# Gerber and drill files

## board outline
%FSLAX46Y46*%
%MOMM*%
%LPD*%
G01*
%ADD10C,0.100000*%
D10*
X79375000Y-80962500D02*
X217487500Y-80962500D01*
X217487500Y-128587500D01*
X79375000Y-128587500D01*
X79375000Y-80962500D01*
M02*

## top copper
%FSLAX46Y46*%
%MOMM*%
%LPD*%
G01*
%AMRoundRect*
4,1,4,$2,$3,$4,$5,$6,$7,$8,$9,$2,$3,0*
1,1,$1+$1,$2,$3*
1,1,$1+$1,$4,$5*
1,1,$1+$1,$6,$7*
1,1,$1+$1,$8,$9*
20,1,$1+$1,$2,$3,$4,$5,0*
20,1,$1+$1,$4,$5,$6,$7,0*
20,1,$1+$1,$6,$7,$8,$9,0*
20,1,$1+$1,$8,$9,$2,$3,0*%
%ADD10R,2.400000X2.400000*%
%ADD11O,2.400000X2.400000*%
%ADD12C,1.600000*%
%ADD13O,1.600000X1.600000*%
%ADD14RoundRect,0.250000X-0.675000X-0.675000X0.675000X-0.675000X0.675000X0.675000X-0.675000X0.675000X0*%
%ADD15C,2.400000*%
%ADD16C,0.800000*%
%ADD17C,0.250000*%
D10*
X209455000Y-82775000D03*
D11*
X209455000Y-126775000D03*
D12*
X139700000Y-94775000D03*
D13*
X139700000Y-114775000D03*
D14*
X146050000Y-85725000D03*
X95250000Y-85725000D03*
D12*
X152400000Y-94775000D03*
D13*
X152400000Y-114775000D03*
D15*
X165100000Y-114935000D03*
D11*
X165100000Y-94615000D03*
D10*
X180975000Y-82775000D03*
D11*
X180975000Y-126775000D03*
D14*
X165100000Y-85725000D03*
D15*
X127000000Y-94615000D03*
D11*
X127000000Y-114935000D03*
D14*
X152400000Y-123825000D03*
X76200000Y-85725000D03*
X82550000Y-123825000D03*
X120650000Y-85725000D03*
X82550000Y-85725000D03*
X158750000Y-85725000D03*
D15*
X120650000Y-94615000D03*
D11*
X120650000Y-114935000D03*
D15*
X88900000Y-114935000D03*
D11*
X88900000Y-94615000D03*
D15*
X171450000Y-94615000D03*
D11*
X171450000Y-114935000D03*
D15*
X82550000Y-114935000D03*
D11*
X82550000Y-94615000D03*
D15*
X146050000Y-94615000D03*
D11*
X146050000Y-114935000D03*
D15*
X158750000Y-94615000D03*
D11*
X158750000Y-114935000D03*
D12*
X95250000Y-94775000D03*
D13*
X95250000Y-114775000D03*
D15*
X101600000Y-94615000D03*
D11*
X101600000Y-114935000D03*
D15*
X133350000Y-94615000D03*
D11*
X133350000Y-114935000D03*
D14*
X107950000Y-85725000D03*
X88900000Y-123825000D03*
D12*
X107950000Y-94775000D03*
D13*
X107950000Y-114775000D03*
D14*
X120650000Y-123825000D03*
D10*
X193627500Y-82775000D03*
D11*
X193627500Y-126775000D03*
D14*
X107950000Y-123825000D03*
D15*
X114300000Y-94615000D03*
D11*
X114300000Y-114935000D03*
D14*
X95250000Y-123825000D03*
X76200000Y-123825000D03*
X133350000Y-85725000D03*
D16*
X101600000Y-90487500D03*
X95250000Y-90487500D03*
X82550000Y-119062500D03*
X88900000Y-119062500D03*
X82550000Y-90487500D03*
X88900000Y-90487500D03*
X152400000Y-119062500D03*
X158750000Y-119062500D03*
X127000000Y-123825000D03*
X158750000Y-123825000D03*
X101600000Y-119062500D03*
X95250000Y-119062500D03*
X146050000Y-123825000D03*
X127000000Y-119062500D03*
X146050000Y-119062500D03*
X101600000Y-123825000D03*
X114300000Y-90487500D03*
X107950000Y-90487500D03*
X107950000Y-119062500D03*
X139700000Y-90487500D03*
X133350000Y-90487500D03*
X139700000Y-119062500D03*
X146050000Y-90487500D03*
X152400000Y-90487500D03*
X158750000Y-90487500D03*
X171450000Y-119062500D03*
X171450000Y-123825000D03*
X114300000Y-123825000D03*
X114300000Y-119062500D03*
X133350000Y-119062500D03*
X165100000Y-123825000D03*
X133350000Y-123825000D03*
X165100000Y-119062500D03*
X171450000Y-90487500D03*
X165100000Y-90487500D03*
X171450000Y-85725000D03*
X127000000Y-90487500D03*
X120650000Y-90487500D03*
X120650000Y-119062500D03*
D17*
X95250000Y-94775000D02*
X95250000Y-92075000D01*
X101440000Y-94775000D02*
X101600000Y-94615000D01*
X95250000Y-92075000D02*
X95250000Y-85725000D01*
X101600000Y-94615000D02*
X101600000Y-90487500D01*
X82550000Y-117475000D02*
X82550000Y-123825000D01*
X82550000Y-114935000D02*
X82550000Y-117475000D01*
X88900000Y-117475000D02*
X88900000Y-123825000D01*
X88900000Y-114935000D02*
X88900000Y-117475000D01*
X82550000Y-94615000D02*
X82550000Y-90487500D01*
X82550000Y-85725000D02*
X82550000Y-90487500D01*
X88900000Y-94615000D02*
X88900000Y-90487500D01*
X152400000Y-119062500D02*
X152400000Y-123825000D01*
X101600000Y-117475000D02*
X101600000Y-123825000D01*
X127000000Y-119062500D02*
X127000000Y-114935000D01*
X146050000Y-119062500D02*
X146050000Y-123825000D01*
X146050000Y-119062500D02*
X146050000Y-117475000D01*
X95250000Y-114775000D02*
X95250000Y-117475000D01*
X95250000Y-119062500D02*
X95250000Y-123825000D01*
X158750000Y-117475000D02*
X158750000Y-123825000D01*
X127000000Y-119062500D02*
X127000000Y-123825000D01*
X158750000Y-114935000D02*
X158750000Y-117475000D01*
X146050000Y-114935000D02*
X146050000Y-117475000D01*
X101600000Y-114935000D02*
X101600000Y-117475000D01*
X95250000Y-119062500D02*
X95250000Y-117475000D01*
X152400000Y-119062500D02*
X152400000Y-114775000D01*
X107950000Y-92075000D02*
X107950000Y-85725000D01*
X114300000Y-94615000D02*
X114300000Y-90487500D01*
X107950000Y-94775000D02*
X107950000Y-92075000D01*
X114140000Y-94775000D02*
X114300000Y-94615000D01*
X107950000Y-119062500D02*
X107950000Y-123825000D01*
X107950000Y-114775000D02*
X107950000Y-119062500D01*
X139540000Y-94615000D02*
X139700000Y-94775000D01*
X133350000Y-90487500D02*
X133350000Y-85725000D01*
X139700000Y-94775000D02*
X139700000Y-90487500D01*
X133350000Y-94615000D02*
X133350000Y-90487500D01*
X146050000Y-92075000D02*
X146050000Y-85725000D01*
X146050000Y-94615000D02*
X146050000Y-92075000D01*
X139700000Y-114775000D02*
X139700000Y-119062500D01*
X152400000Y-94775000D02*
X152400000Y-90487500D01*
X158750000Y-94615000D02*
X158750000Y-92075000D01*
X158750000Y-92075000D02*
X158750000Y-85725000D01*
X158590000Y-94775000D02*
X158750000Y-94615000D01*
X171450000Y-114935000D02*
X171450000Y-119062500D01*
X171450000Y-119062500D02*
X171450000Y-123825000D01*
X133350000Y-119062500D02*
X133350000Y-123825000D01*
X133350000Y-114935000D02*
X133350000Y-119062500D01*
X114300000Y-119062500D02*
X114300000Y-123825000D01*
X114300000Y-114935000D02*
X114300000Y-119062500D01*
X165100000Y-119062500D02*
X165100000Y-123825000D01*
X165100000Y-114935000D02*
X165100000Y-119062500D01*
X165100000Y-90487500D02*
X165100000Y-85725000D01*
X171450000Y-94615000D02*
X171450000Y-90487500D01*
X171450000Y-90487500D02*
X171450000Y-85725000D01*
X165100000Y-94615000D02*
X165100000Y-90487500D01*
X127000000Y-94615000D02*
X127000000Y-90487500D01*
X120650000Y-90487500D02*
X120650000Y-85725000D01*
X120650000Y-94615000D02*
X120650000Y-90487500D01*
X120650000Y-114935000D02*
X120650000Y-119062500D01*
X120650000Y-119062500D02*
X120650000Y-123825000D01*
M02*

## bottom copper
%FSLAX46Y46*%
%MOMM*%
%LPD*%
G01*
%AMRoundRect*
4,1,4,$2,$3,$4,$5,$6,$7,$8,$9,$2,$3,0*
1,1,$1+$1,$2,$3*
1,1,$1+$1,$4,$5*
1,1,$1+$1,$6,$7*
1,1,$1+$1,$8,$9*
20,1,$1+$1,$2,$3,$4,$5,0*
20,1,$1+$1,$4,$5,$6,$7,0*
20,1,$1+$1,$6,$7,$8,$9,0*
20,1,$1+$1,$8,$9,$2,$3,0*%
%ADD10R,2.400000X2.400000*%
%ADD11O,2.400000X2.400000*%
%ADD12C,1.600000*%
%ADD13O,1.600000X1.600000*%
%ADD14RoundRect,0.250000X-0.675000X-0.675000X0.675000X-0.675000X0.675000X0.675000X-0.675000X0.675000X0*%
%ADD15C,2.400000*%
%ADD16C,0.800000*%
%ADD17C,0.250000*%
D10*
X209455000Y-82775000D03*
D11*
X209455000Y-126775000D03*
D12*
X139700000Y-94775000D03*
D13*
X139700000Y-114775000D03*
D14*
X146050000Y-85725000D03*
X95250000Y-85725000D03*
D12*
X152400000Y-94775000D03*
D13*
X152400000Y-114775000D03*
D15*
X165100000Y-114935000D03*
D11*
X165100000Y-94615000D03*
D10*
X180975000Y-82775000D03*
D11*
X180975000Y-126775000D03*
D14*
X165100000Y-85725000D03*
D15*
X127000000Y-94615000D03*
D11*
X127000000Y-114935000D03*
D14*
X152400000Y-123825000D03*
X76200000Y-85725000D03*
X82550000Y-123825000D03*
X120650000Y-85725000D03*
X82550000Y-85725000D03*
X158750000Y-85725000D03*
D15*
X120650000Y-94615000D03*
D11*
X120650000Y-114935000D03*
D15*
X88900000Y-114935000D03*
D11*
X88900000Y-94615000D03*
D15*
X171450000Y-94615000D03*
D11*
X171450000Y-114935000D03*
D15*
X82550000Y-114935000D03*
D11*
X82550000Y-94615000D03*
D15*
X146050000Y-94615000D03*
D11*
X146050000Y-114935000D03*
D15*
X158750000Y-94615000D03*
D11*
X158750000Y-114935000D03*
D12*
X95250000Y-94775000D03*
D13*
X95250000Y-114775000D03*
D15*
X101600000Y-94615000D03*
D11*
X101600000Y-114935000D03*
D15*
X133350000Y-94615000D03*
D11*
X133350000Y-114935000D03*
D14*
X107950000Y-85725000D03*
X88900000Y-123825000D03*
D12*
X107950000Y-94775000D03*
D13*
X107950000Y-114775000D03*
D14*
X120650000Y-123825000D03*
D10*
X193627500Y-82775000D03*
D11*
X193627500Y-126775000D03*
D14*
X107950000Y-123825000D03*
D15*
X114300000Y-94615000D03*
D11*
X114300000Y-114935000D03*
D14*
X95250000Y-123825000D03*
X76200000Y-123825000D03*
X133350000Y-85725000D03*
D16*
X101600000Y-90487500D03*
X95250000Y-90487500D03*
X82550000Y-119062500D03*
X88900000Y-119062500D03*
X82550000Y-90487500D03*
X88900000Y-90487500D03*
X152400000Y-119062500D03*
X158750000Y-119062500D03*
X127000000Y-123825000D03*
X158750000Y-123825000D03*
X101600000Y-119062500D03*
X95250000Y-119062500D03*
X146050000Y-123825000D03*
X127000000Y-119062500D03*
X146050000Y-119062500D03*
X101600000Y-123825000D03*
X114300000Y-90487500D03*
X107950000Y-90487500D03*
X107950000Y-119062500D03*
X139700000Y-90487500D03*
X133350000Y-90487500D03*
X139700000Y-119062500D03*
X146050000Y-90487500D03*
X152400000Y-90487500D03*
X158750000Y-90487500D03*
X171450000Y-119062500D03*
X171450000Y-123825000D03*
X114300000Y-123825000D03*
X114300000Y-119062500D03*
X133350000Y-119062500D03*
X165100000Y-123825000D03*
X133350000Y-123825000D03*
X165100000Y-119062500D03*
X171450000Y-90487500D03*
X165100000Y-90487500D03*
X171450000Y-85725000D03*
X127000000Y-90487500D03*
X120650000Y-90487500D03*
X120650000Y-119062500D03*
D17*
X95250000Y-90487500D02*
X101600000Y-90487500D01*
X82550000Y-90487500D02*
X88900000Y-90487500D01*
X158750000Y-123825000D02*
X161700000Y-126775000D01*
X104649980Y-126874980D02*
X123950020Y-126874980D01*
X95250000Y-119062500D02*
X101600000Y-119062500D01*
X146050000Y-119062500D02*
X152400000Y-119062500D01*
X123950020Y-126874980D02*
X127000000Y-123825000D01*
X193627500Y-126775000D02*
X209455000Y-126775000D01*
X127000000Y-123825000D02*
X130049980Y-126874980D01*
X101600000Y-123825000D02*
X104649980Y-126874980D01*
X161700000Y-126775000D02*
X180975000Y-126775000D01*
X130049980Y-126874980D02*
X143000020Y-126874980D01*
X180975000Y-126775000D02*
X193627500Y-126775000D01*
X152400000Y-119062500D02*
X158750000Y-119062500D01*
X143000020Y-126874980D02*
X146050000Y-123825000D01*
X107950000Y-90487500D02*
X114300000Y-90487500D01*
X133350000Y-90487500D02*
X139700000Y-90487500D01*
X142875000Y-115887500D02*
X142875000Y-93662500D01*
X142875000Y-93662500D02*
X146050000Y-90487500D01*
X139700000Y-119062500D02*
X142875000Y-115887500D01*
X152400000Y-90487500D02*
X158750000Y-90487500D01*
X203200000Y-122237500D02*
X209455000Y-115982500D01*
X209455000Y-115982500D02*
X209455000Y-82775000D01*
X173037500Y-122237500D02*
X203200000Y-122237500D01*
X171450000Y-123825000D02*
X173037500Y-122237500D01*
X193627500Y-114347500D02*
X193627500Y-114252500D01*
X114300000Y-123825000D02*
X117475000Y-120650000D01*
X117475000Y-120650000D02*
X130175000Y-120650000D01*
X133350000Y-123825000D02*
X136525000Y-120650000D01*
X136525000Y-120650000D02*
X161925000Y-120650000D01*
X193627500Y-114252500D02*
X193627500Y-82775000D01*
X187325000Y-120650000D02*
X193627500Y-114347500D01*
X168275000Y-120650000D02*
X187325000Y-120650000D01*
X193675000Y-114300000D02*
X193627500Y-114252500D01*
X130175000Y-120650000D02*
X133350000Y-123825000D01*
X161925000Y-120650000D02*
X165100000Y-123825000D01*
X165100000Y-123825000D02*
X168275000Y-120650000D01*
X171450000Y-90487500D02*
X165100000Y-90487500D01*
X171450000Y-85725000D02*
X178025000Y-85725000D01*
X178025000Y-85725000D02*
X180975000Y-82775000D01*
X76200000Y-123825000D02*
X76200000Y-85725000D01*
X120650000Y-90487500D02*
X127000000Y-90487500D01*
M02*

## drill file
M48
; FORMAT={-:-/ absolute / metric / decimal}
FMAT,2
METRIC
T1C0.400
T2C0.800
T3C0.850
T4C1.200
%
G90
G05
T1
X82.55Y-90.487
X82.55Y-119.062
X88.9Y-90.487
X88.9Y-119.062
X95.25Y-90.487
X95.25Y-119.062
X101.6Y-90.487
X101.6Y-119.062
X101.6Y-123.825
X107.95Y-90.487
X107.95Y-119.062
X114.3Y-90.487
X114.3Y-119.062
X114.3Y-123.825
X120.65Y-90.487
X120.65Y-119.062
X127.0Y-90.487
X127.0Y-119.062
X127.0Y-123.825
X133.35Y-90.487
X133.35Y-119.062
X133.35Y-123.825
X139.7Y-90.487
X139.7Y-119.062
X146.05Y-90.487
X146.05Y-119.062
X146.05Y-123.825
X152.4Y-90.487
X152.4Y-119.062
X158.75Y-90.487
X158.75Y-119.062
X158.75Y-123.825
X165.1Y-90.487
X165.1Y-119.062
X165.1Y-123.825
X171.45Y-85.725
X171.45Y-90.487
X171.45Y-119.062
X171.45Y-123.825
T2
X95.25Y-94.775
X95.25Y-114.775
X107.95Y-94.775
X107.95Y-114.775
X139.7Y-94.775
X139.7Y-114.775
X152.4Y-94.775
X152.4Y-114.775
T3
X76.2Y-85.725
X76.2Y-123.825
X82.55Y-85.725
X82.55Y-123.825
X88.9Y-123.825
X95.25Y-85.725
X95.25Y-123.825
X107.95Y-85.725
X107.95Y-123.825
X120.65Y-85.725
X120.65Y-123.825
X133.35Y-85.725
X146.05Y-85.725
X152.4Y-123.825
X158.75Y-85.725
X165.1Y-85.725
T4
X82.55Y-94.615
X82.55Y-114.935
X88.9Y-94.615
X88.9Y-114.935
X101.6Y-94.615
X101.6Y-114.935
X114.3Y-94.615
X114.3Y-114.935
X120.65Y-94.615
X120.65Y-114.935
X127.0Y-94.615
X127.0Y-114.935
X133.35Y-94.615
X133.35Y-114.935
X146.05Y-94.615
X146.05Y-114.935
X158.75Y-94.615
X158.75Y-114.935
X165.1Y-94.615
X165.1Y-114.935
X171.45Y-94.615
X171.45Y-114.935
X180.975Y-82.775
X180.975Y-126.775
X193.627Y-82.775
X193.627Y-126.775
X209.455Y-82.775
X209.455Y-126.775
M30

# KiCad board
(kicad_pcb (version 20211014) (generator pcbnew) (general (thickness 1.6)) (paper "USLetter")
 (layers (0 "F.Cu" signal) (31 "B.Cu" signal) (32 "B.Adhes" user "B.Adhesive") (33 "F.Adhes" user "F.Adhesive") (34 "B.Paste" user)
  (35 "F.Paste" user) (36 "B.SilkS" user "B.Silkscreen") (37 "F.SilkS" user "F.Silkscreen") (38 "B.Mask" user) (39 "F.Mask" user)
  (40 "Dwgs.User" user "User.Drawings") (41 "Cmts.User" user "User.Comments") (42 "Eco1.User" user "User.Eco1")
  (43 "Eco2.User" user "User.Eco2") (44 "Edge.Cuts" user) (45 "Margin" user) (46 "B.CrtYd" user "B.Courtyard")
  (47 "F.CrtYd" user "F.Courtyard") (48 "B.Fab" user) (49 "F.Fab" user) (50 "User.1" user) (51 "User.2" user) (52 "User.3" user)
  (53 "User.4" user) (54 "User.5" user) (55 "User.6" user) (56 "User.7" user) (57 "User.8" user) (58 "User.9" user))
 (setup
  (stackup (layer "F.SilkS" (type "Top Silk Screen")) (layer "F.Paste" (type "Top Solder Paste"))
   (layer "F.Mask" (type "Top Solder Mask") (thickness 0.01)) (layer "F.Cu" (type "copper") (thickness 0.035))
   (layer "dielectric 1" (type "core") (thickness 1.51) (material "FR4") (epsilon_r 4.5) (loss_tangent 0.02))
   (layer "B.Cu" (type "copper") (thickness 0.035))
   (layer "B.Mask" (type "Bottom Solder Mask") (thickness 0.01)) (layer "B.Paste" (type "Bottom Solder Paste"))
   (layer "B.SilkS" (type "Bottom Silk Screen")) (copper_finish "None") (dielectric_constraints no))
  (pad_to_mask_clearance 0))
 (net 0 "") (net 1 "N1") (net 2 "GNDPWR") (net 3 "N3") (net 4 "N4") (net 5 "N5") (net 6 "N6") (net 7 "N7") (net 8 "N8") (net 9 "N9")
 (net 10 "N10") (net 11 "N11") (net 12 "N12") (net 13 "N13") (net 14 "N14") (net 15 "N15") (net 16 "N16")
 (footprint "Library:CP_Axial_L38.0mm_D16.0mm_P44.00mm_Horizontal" (layer "F.Cu") (at 209.455 82.775 -90)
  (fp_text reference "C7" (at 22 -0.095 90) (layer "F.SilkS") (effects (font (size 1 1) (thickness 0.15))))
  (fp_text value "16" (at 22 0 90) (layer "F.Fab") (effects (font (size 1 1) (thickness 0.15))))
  (pad "1" thru_hole rect (at 0 0 270) (size 2.4 2.4) (drill 1.2) (layers *.Cu *.Mask) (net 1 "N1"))
  (pad "2" thru_hole oval (at 44 0 270) (size 2.4 2.4) (drill 1.2) (layers *.Cu *.Mask) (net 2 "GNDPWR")))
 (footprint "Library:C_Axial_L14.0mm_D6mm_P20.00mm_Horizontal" (layer "F.Cu") (at 139.7 94.775 -90)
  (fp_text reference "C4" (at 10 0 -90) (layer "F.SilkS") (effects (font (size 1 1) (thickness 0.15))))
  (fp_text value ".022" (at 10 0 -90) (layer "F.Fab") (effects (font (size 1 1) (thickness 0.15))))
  (pad "1" thru_hole circle (at 0 0 270) (size 1.6 1.6) (drill 0.8) (layers *.Cu *.Mask) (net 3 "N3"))
  (pad "2" thru_hole oval (at 20 0 270) (size 1.6 1.6) (drill 0.8) (layers *.Cu *.Mask) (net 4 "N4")))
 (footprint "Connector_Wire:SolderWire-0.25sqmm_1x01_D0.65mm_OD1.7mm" (layer "F.Cu") (at 146.05 85.725)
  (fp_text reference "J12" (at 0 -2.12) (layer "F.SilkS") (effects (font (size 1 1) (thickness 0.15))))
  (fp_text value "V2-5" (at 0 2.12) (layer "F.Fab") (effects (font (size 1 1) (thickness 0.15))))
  (pad "1" thru_hole roundrect (at 0 0) (size 1.85 1.85) (drill 0.85) (layers *.Cu *.Mask) (roundrect_rratio 0.135135) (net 4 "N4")))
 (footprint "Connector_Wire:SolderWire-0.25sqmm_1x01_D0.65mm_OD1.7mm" (layer "F.Cu") (at 95.25 85.725)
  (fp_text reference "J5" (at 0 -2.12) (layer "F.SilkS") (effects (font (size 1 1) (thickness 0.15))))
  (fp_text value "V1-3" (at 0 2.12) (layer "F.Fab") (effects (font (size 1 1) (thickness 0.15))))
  (pad "1" thru_hole roundrect (at 0 0) (size 1.85 1.85) (drill 0.85) (layers *.Cu *.Mask) (roundrect_rratio 0.135135) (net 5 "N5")))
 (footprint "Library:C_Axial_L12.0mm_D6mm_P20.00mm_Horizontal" (layer "F.Cu") (at 152.4 94.775 -90)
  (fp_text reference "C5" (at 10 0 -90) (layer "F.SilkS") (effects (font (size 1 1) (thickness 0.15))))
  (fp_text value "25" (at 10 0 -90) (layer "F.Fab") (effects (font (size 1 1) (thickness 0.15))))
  (pad "1" thru_hole circle (at 0 0 270) (size 1.6 1.6) (drill 0.8) (layers *.Cu *.Mask) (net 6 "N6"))
  (pad "2" thru_hole oval (at 20 0 270) (size 1.6 1.6) (drill 0.8) (layers *.Cu *.Mask) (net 2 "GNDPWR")))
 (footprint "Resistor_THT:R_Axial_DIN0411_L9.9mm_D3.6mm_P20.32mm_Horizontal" (layer "F.Cu") (at 165.1 114.935 90)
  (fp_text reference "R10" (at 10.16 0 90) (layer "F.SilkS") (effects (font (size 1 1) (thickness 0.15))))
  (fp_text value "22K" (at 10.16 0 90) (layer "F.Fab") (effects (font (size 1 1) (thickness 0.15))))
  (pad "1" thru_hole circle (at 0 0 90) (size 2.4 2.4) (drill 1.2) (layers *.Cu *.Mask) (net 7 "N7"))
  (pad "2" thru_hole oval (at 20.32 0 90) (size 2.4 2.4) (drill 1.2) (layers *.Cu *.Mask) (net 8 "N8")))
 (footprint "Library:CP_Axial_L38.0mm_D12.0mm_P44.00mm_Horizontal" (layer "F.Cu") (at 180.975 82.775 -90)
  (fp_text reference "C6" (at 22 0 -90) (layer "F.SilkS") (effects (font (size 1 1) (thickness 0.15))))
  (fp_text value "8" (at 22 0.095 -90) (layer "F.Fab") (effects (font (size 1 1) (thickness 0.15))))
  (pad "1" thru_hole rect (at 0 0 270) (size 2.4 2.4) (drill 1.2) (layers *.Cu *.Mask) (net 8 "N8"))
  (pad "2" thru_hole oval (at 44 0 270) (size 2.4 2.4) (drill 1.2) (layers *.Cu *.Mask) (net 2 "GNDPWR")))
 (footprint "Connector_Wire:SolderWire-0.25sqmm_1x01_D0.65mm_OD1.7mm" (layer "F.Cu") (at 165.1 85.725)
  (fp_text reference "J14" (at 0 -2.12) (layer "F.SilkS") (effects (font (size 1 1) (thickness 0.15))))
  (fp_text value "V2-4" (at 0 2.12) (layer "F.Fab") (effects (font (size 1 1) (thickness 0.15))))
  (pad "1" thru_hole roundrect (at 0 0) (size 1.85 1.85) (drill 0.85) (layers *.Cu *.Mask) (roundrect_rratio 0.135135) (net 8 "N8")))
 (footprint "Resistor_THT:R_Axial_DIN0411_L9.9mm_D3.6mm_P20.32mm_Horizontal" (layer "F.Cu") (at 127 94.615 -90)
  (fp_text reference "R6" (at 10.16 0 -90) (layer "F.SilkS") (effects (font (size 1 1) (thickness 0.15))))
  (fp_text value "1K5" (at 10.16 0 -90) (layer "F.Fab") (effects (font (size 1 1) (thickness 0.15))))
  (pad "1" thru_hole circle (at 0 0 270) (size 2.4 2.4) (drill 1.2) (layers *.Cu *.Mask) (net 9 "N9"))
  (pad "2" thru_hole oval (at 20.32 0 270) (size 2.4 2.4) (drill 1.2) (layers *.Cu *.Mask) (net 2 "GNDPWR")))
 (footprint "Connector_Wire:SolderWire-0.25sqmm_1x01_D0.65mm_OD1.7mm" (layer "F.Cu") (at 152.4 123.825)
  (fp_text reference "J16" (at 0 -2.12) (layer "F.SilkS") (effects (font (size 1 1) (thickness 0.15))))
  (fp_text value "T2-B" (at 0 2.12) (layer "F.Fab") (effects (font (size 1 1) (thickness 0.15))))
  (pad "1" thru_hole roundrect (at 0 0) (size 1.85 1.85) (drill 0.85) (layers *.Cu *.Mask) (roundrect_rratio 0.135135) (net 2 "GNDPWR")))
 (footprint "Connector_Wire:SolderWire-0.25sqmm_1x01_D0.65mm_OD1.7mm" (layer "F.Cu") (at 76.2 85.725)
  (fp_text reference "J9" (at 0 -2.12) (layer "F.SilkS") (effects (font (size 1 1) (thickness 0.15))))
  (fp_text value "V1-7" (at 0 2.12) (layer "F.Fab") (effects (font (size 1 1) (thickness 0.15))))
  (pad "1" thru_hole roundrect (at 0 0) (size 1.85 1.85) (drill 0.85) (layers *.Cu *.Mask) (roundrect_rratio 0.135135) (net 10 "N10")))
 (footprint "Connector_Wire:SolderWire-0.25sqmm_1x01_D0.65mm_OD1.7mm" (layer "F.Cu") (at 82.55 123.825)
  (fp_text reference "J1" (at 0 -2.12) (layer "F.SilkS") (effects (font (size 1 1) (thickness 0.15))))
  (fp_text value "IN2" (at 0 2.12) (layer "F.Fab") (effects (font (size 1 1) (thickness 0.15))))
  (pad "1" thru_hole roundrect (at 0 0) (size 1.85 1.85) (drill 0.85) (layers *.Cu *.Mask) (roundrect_rratio 0.135135) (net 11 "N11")))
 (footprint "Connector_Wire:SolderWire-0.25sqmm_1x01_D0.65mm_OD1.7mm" (layer "F.Cu") (at 120.65 85.725)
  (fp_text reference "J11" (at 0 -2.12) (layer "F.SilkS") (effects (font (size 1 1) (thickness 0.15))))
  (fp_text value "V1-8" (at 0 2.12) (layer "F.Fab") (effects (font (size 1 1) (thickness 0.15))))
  (pad "1" thru_hole roundrect (at 0 0) (size 1.85 1.85) (drill 0.85) (layers *.Cu *.Mask) (roundrect_rratio 0.135135) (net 9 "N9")))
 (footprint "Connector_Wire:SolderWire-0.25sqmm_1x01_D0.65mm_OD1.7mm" (layer "F.Cu") (at 82.55 85.725)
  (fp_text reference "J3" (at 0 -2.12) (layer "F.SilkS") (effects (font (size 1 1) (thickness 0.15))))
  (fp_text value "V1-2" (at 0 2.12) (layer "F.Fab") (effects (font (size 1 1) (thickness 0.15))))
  (pad "1" thru_hole roundrect (at 0 0) (size 1.85 1.85) (drill 0.85) (layers *.Cu *.Mask) (roundrect_rratio 0.135135) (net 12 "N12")))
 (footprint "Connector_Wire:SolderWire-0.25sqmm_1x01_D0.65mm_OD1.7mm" (layer "F.Cu") (at 158.75 85.725)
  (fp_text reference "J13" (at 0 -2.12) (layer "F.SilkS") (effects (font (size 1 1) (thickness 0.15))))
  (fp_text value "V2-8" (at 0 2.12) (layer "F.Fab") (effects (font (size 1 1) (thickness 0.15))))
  (pad "1" thru_hole roundrect (at 0 0) (size 1.85 1.85) (drill 0.85) (layers *.Cu *.Mask) (roundrect_rratio 0.135135) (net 6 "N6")))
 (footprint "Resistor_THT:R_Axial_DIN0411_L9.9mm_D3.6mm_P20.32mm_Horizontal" (layer "F.Cu") (at 120.65 94.615 -90)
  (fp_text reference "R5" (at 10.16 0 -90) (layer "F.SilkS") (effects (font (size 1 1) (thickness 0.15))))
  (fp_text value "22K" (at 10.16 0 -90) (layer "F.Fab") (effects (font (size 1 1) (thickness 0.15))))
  (pad "1" thru_hole circle (at 0 0 270) (size 2.4 2.4) (drill 1.2) (layers *.Cu *.Mask) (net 9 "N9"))
  (pad "2" thru_hole oval (at 20.32 0 270) (size 2.4 2.4) (drill 1.2) (layers *.Cu *.Mask) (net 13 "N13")))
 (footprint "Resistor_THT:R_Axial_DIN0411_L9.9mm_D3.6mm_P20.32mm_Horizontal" (layer "F.Cu") (at 88.9 114.935 90)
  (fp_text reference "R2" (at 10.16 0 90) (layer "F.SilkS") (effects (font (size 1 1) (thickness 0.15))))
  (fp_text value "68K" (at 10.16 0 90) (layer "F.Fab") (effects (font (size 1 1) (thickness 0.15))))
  (pad "1" thru_hole circle (at 0 0 90) (size 2.4 2.4) (drill 1.2) (layers *.Cu *.Mask) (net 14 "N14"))
  (pad "2" thru_hole oval (at 20.32 0 90) (size 2.4 2.4) (drill 1.2) (layers *.Cu *.Mask) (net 12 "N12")))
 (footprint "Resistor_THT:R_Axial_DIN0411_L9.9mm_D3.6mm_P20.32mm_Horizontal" (layer "F.Cu") (at 171.45 94.615 -90)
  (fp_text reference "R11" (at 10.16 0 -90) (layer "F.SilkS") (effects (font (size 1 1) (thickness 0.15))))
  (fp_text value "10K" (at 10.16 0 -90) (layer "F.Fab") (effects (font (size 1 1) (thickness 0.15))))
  (pad "1" thru_hole circle (at 0 0 270) (size 2.4 2.4) (drill 1.2) (layers *.Cu *.Mask) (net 8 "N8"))
  (pad "2" thru_hole oval (at 20.32 0 270) (size 2.4 2.4) (drill 1.2) (layers *.Cu *.Mask) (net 1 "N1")))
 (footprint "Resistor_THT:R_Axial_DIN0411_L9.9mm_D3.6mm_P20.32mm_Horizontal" (layer "F.Cu") (at 82.55 114.935 90)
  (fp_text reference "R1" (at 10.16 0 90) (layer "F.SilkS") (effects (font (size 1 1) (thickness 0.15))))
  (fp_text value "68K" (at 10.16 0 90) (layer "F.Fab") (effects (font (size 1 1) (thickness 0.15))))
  (pad "1" thru_hole circle (at 0 0 90) (size 2.4 2.4) (drill 1.2) (layers *.Cu *.Mask) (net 11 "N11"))
  (pad "2" thru_hole oval (at 20.32 0 90) (size 2.4 2.4) (drill 1.2) (layers *.Cu *.Mask) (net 12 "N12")))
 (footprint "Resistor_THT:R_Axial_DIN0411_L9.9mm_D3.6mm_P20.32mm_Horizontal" (layer "F.Cu") (at 146.05 94.615 -90)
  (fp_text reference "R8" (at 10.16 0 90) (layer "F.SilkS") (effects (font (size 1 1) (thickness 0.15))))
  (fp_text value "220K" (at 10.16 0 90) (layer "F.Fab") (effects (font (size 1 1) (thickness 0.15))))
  (pad "1" thru_hole circle (at 0 0 270) (size 2.4 2.4) (drill 1.2) (layers *.Cu *.Mask) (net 4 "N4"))
  (pad "2" thru_hole oval (at 20.32 0 270) (size 2.4 2.4) (drill 1.2) (layers *.Cu *.Mask) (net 2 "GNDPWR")))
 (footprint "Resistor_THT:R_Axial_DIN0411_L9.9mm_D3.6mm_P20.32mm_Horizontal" (layer "F.Cu") (at 158.75 94.615 -90)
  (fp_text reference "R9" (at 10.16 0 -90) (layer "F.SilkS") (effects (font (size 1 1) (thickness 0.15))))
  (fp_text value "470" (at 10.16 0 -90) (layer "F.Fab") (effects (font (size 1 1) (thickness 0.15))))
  (pad "1" thru_hole circle (at 0 0 270) (size 2.4 2.4) (drill 1.2) (layers *.Cu *.Mask) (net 6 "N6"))
  (pad "2" thru_hole oval (at 20.32 0 270) (size 2.4 2.4) (drill 1.2) (layers *.Cu *.Mask) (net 2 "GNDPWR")))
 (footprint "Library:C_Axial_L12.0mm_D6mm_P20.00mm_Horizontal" (layer "F.Cu") (at 95.25 94.775 -90)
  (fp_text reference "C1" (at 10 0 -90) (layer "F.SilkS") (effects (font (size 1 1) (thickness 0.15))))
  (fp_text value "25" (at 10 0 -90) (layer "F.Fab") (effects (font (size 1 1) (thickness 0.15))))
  (pad "1" thru_hole circle (at 0 0 270) (size 1.6 1.6) (drill 0.8) (layers *.Cu *.Mask) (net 5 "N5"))
  (pad "2" thru_hole oval (at 20 0 270) (size 1.6 1.6) (drill 0.8) (layers *.Cu *.Mask) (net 2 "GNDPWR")))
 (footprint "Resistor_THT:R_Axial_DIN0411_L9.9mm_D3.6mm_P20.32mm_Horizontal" (layer "F.Cu") (at 101.6 94.615 -90)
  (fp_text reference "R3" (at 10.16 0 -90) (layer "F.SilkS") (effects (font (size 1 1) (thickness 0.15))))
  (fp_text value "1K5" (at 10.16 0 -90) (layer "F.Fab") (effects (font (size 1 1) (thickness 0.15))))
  (pad "1" thru_hole circle (at 0 0 270) (size 2.4 2.4) (drill 1.2) (layers *.Cu *.Mask) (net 5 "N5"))
  (pad "2" thru_hole oval (at 20.32 0 270) (size 2.4 2.4) (drill 1.2) (layers *.Cu *.Mask) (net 2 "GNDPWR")))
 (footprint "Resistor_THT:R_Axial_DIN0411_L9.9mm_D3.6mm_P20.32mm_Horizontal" (layer "F.Cu") (at 133.35 94.615 -90)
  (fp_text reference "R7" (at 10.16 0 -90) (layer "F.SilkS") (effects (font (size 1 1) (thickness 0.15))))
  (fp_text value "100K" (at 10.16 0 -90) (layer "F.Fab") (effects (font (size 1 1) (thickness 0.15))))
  (pad "1" thru_hole circle (at 0 0 270) (size 2.4 2.4) (drill 1.2) (layers *.Cu *.Mask) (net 3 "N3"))
  (pad "2" thru_hole oval (at 20.32 0 270) (size 2.4 2.4) (drill 1.2) (layers *.Cu *.Mask) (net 7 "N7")))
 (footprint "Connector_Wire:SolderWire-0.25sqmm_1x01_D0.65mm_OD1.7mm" (layer "F.Cu") (at 107.95 85.725)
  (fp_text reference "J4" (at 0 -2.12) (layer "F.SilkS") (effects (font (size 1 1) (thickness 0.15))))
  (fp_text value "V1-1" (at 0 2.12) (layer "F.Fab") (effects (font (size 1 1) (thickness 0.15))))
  (pad "1" thru_hole roundrect (at 0 0) (size 1.85 1.85) (drill 0.85) (layers *.Cu *.Mask) (roundrect_rratio 0.135135) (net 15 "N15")))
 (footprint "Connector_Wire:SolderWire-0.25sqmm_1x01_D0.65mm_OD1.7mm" (layer "F.Cu") (at 88.9 123.825)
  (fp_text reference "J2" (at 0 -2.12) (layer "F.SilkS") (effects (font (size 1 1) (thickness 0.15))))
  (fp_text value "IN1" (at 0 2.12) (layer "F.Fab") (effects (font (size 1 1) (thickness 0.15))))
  (pad "1" thru_hole roundrect (at 0 0) (size 1.85 1.85) (drill 0.85) (layers *.Cu *.Mask) (roundrect_rratio 0.135135) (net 14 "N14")))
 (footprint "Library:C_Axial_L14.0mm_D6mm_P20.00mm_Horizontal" (layer "F.Cu") (at 107.95 94.775 -90)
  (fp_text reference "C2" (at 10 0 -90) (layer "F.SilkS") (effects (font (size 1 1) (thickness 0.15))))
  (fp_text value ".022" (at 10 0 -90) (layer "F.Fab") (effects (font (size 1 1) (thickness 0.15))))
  (pad "1" thru_hole circle (at 0 0 270) (size 1.6 1.6) (drill 0.8) (layers *.Cu *.Mask) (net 15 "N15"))
  (pad "2" thru_hole oval (at 20 0 270) (size 1.6 1.6) (drill 0.8) (layers *.Cu *.Mask) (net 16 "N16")))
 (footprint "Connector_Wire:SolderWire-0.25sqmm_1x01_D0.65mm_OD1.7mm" (layer "F.Cu") (at 120.65 123.825)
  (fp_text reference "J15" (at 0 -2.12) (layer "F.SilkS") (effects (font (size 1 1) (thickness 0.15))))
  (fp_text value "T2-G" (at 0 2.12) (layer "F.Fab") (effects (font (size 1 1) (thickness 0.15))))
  (pad "1" thru_hole roundrect (at 0 0) (size 1.85 1.85) (drill 0.85) (layers *.Cu *.Mask) (roundrect_rratio 0.135135) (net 13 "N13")))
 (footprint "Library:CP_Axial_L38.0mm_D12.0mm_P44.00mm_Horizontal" (layer "F.Cu") (at 193.6275 82.775 -90)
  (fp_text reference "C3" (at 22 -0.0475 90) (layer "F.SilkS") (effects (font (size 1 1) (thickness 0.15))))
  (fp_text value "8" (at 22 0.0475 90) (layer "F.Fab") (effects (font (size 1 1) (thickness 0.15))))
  (pad "1" thru_hole rect (at 0 0 270) (size 2.4 2.4) (drill 1.2) (layers *.Cu *.Mask) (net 7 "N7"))
  (pad "2" thru_hole oval (at 44 0 270) (size 2.4 2.4) (drill 1.2) (layers *.Cu *.Mask) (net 2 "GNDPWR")))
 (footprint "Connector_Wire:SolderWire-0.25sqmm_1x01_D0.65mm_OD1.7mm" (layer "F.Cu") (at 107.95 123.825)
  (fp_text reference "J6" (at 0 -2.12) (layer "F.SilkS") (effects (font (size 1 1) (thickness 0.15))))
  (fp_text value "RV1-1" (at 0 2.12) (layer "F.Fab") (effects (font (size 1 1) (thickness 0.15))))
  (pad "1" thru_hole roundrect (at 0 0) (size 1.85 1.85) (drill 0.85) (layers *.Cu *.Mask) (roundrect_rratio 0.135135) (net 16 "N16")))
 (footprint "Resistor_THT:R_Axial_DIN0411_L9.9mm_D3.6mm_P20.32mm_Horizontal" (layer "F.Cu") (at 114.3 94.615 -90)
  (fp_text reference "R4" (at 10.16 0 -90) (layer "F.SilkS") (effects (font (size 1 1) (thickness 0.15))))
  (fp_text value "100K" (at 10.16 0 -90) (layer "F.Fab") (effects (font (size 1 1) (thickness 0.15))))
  (pad "1" thru_hole circle (at 0 0 270) (size 2.4 2.4) (drill 1.2) (layers *.Cu *.Mask) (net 15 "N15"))
  (pad "2" thru_hole oval (at 20.32 0 270) (size 2.4 2.4) (drill 1.2) (layers *.Cu *.Mask) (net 7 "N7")))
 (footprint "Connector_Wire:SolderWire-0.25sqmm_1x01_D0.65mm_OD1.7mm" (layer "F.Cu") (at 95.25 123.825)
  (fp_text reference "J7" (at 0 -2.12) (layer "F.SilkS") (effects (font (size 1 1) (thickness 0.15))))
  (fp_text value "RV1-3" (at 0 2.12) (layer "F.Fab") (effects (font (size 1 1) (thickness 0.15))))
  (pad "1" thru_hole roundrect (at 0 0) (size 1.85 1.85) (drill 0.85) (layers *.Cu *.Mask) (roundrect_rratio 0.135135) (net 2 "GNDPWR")))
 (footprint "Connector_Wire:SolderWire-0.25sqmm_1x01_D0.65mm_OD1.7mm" (layer "F.Cu") (at 76.2 123.825)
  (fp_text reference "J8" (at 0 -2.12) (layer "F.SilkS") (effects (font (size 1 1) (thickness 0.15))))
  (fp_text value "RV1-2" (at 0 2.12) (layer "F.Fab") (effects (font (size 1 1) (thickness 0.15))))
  (pad "1" thru_hole roundrect (at 0 0) (size 1.85 1.85) (drill 0.85) (layers *.Cu *.Mask) (roundrect_rratio 0.135135) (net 10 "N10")))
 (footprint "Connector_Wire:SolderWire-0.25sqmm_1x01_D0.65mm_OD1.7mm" (layer "F.Cu") (at 133.35 85.725)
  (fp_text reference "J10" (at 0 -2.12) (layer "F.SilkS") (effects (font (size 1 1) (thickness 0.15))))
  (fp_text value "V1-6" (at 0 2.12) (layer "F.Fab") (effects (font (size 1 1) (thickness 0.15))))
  (pad "1" thru_hole roundrect (at 0 0) (size 1.85 1.85) (drill 0.85) (layers *.Cu *.Mask) (roundrect_rratio 0.135135) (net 3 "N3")))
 (gr_rect (start 217.4875 80.9625) (end 79.375 128.5875) (layer "Edge.Cuts") (width 0.1) (fill none))
 (segment (start 95.25 94.775) (end 95.25 92.075) (width 0.25) (layer "F.Cu") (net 5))
 (segment (start 101.44 94.775) (end 101.6 94.615) (width 0.25) (layer "F.Cu") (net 5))
 (segment (start 95.25 92.075) (end 95.25 85.725) (width 0.25) (layer "F.Cu") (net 5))
 (segment (start 101.6 94.615) (end 101.6 90.4875) (width 0.25) (layer "F.Cu") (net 5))
 (via (at 101.6 90.4875) (size 0.8) (drill 0.4) (layers "F.Cu" "B.Cu") (free) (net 5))
 (via (at 95.25 90.4875) (size 0.8) (drill 0.4) (layers "F.Cu" "B.Cu") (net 5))
 (segment (start 95.25 90.4875) (end 101.6 90.4875) (width 0.25) (layer "B.Cu") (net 5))
 (segment (start 82.55 117.475) (end 82.55 123.825) (width 0.25) (layer "F.Cu") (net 11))
 (segment (start 82.55 114.935) (end 82.55 117.475) (width 0.25) (layer "F.Cu") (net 11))
 (via (at 82.55 119.0625) (size 0.8) (drill 0.4) (layers "F.Cu" "B.Cu") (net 11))
 (segment (start 88.9 117.475) (end 88.9 123.825) (width 0.25) (layer "F.Cu") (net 14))
 (segment (start 88.9 114.935) (end 88.9 117.475) (width 0.25) (layer "F.Cu") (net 14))
 (via (at 88.9 119.0625) (size 0.8) (drill 0.4) (layers "F.Cu" "B.Cu") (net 14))
 (segment (start 82.55 94.615) (end 82.55 90.4875) (width 0.25) (layer "F.Cu") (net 12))
 (segment (start 82.55 85.725) (end 82.55 90.4875) (width 0.25) (layer "F.Cu") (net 12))
 (segment (start 88.9 94.615) (end 88.9 90.4875) (width 0.25) (layer "F.Cu") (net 12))
 (via (at 82.55 90.4875) (size 0.8) (drill 0.4) (layers "F.Cu" "B.Cu") (free) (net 12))
 (via (at 88.9 90.4875) (size 0.8) (drill 0.4) (layers "F.Cu" "B.Cu") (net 12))
 (segment (start 82.55 90.4875) (end 88.9 90.4875) (width 0.25) (layer "B.Cu") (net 12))
 (segment (start 152.4 119.0625) (end 152.4 123.825) (width 0.25) (layer "F.Cu") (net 2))
 (segment (start 101.6 117.475) (end 101.6 123.825) (width 0.25) (layer "F.Cu") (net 2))
 (segment (start 127 119.0625) (end 127 114.935) (width 0.25) (layer "F.Cu") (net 2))
 (segment (start 146.05 119.0625) (end 146.05 123.825) (width 0.25) (layer "F.Cu") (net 2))
 (segment (start 146.05 119.0625) (end 146.05 117.475) (width 0.25) (layer "F.Cu") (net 2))
 (segment (start 95.25 114.775) (end 95.25 117.475) (width 0.25) (layer "F.Cu") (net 2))
 (segment (start 95.25 119.0625) (end 95.25 123.825) (width 0.25) (layer "F.Cu") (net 2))
 (segment (start 158.75 117.475) (end 158.75 123.825) (width 0.25) (layer "F.Cu") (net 2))
 (segment (start 127 119.0625) (end 127 123.825) (width 0.25) (layer "F.Cu") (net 2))
 (segment (start 158.75 114.935) (end 158.75 117.475) (width 0.25) (layer "F.Cu") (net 2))
 (segment (start 146.05 114.935) (end 146.05 117.475) (width 0.25) (layer "F.Cu") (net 2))
 (segment (start 101.6 114.935) (end 101.6 117.475) (width 0.25) (layer "F.Cu") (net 2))
 (segment (start 95.25 119.0625) (end 95.25 117.475) (width 0.25) (layer "F.Cu") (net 2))
 (segment (start 152.4 119.0625) (end 152.4 114.775) (width 0.25) (layer "F.Cu") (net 2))
 (via (at 152.4 119.0625) (size 0.8) (drill 0.4) (layers "F.Cu" "B.Cu") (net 2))
 (via (at 158.75 119.0625) (size 0.8) (drill 0.4) (layers "F.Cu" "B.Cu") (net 2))
 (via (at 127 123.825) (size 0.8) (drill 0.4) (layers "F.Cu" "B.Cu") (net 2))
 (via (at 158.75 123.825) (size 0.8) (drill 0.4) (layers "F.Cu" "B.Cu") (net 2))
 (via (at 101.6 119.0625) (size 0.8) (drill 0.4) (layers "F.Cu" "B.Cu") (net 2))
 (via (at 95.25 119.0625) (size 0.8) (drill 0.4) (layers "F.Cu" "B.Cu") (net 2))
 (via (at 146.05 123.825) (size 0.8) (drill 0.4) (layers "F.Cu" "B.Cu") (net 2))
 (via (at 127 119.0625) (size 0.8) (drill 0.4) (layers "F.Cu" "B.Cu") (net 2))
 (via (at 146.05 119.0625) (size 0.8) (drill 0.4) (layers "F.Cu" "B.Cu") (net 2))
 (via (at 101.6 123.825) (size 0.8) (drill 0.4) (layers "F.Cu" "B.Cu") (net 2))
 (segment (start 158.75 123.825) (end 161.7 126.775) (width 0.25) (layer "B.Cu") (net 2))
 (segment (start 104.64998 126.87498) (end 123.95002 126.87498) (width 0.25) (layer "B.Cu") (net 2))
 (segment (start 95.25 119.0625) (end 101.6 119.0625) (width 0.25) (layer "B.Cu") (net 2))
 (segment (start 146.05 119.0625) (end 152.4 119.0625) (width 0.25) (layer "B.Cu") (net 2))
 (segment (start 123.95002 126.87498) (end 127 123.825) (width 0.25) (layer "B.Cu") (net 2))
 (segment (start 193.6275 126.775) (end 209.455 126.775) (width 0.25) (layer "B.Cu") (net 2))
 (segment (start 127 123.825) (end 130.04998 126.87498) (width 0.25) (layer "B.Cu") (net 2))
 (segment (start 101.6 123.825) (end 104.64998 126.87498) (width 0.25) (layer "B.Cu") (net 2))
 (segment (start 161.7 126.775) (end 180.975 126.775) (width 0.25) (layer "B.Cu") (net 2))
 (segment (start 130.04998 126.87498) (end 143.00002 126.87498) (width 0.25) (layer "B.Cu") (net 2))
 (segment (start 180.975 126.775) (end 193.6275 126.775) (width 0.25) (layer "B.Cu") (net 2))
 (segment (start 152.4 119.0625) (end 158.75 119.0625) (width 0.25) (layer "B.Cu") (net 2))
 (segment (start 143.00002 126.87498) (end 146.05 123.825) (width 0.25) (layer "B.Cu") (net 2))
 (segment (start 107.95 92.075) (end 107.95 85.725) (width 0.25) (layer "F.Cu") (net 15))
 (segment (start 114.3 94.615) (end 114.3 90.4875) (width 0.25) (layer "F.Cu") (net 15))
 (segment (start 107.95 94.775) (end 107.95 92.075) (width 0.25) (layer "F.Cu") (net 15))
 (segment (start 114.14 94.775) (end 114.3 94.615) (width 0.25) (layer "F.Cu") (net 15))
 (via (at 114.3 90.4875) (size 0.8) (drill 0.4) (layers "F.Cu" "B.Cu") (free) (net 15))
 (via (at 107.95 90.4875) (size 0.8) (drill 0.4) (layers "F.Cu" "B.Cu") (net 15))
 (segment (start 107.95 90.4875) (end 114.3 90.4875) (width 0.25) (layer "B.Cu") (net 15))
 (segment (start 107.95 119.0625) (end 107.95 123.825) (width 0.25) (layer "F.Cu") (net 16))
 (segment (start 107.95 114.775) (end 107.95 119.0625) (width 0.25) (layer "F.Cu") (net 16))
 (via (at 107.95 119.0625) (size 0.8) (drill 0.4) (layers "F.Cu" "B.Cu") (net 16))
 (segment (start 139.54 94.615) (end 139.7 94.775) (width 0.25) (layer "F.Cu") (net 3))
 (segment (start 133.35 90.4875) (end 133.35 85.725) (width 0.25) (layer "F.Cu") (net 3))
 (segment (start 139.7 94.775) (end 139.7 90.4875) (width 0.25) (layer "F.Cu") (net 3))
 (segment (start 133.35 94.615) (end 133.35 90.4875) (width 0.25) (layer "F.Cu") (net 3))
 (via (at 139.7 90.4875) (size 0.8) (drill 0.4) (layers "F.Cu" "B.Cu") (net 3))
 (via (at 133.35 90.4875) (size 0.8) (drill 0.4) (layers "F.Cu" "B.Cu") (free) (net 3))
 (segment (start 133.35 90.4875) (end 139.7 90.4875) (width 0.25) (layer "B.Cu") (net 3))
 (segment (start 146.05 92.075) (end 146.05 85.725) (width 0.25) (layer "F.Cu") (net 4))
 (segment (start 146.05 94.615) (end 146.05 92.075) (width 0.25) (layer "F.Cu") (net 4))
 (segment (start 139.7 114.775) (end 139.7 119.0625) (width 0.25) (layer "F.Cu") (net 4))
 (via (at 139.7 119.0625) (size 0.8) (drill 0.4) (layers "F.Cu" "B.Cu") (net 4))
 (via (at 146.05 90.4875) (size 0.8) (drill 0.4) (layers "F.Cu" "B.Cu") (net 4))
 (segment (start 142.875 115.8875) (end 142.875 93.6625) (width 0.25) (layer "B.Cu") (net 4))
 (segment (start 142.875 93.6625) (end 146.05 90.4875) (width 0.25) (layer "B.Cu") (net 4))
 (segment (start 139.7 119.0625) (end 142.875 115.8875) (width 0.25) (layer "B.Cu") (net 4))
 (segment (start 152.4 94.775) (end 152.4 90.4875) (width 0.25) (layer "F.Cu") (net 6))
 (segment (start 158.75 94.615) (end 158.75 92.075) (width 0.25) (layer "F.Cu") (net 6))
 (segment (start 158.75 92.075) (end 158.75 85.725) (width 0.25) (layer "F.Cu") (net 6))
 (segment (start 158.59 94.775) (end 158.75 94.615) (width 0.25) (layer "F.Cu") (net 6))
 (via (at 152.4 90.4875) (size 0.8) (drill 0.4) (layers "F.Cu" "B.Cu") (free) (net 6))
 (via (at 158.75 90.4875) (size 0.8) (drill 0.4) (layers "F.Cu" "B.Cu") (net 6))
 (segment (start 152.4 90.4875) (end 158.75 90.4875) (width 0.25) (layer "B.Cu") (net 6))
 (segment (start 171.45 114.935) (end 171.45 119.0625) (width 0.25) (layer "F.Cu") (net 1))
 (segment (start 171.45 119.0625) (end 171.45 123.825) (width 0.25) (layer "F.Cu") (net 1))
 (via (at 171.45 119.0625) (size 0.8) (drill 0.4) (layers "F.Cu" "B.Cu") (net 1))
 (via (at 171.45 123.825) (size 0.8) (drill 0.4) (layers "F.Cu" "B.Cu") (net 1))
 (segment (start 203.2 122.2375) (end 209.455 115.9825) (width 0.25) (layer "B.Cu") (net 1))
 (segment (start 209.455 115.9825) (end 209.455 82.775) (width 0.25) (layer "B.Cu") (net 1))
 (segment (start 173.0375 122.2375) (end 203.2 122.2375) (width 0.25) (layer "B.Cu") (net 1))
 (segment (start 171.45 123.825) (end 173.0375 122.2375) (width 0.25) (layer "B.Cu") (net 1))
 (segment (start 133.35 119.0625) (end 133.35 123.825) (width 0.25) (layer "F.Cu") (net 7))
 (segment (start 133.35 114.935) (end 133.35 119.0625) (width 0.25) (layer "F.Cu") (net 7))
 (segment (start 114.3 119.0625) (end 114.3 123.825) (width 0.25) (layer "F.Cu") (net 7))
 (segment (start 114.3 114.935) (end 114.3 119.0625) (width 0.25) (layer "F.Cu") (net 7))
 (segment (start 165.1 119.0625) (end 165.1 123.825) (width 0.25) (layer "F.Cu") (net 7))
 (segment (start 165.1 114.935) (end 165.1 119.0625) (width 0.25) (layer "F.Cu") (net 7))
 (via (at 114.3 123.825) (size 0.8) (drill 0.4) (layers "F.Cu" "B.Cu") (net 7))
 (via (at 114.3 119.0625) (size 0.8) (drill 0.4) (layers "F.Cu" "B.Cu") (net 7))
 (via (at 133.35 119.0625) (size 0.8) (drill 0.4) (layers "F.Cu" "B.Cu") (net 7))
 (via (at 165.1 123.825) (size 0.8) (drill 0.4) (layers "F.Cu" "B.Cu") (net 7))
 (via (at 133.35 123.825) (size 0.8) (drill 0.4) (layers "F.Cu" "B.Cu") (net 7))
 (via (at 165.1 119.0625) (size 0.8) (drill 0.4) (layers "F.Cu" "B.Cu") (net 7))
 (segment (start 193.6275 114.3475) (end 193.6275 114.2525) (width 0.25) (layer "B.Cu") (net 7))
 (segment (start 114.3 123.825) (end 117.475 120.65) (width 0.25) (layer "B.Cu") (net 7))
 (segment (start 117.475 120.65) (end 130.175 120.65) (width 0.25) (layer "B.Cu") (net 7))
 (segment (start 133.35 123.825) (end 136.525 120.65) (width 0.25) (layer "B.Cu") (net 7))
 (segment (start 136.525 120.65) (end 161.925 120.65) (width 0.25) (layer "B.Cu") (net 7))
 (segment (start 193.6275 114.2525) (end 193.6275 82.775) (width 0.25) (layer "B.Cu") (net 7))
 (segment (start 187.325 120.65) (end 193.6275 114.3475) (width 0.25) (layer "B.Cu") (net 7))
 (segment (start 168.275 120.65) (end 187.325 120.65) (width 0.25) (layer "B.Cu") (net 7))
 (segment (start 193.675 114.3) (end 193.6275 114.2525) (width 0.25) (layer "B.Cu") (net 7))
 (segment (start 130.175 120.65) (end 133.35 123.825) (width 0.25) (layer "B.Cu") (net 7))
 (segment (start 161.925 120.65) (end 165.1 123.825) (width 0.25) (layer "B.Cu") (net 7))
 (segment (start 165.1 123.825) (end 168.275 120.65) (width 0.25) (layer "B.Cu") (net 7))
 (segment (start 165.1 90.4875) (end 165.1 85.725) (width 0.25) (layer "F.Cu") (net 8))
 (segment (start 171.45 94.615) (end 171.45 90.4875) (width 0.25) (layer "F.Cu") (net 8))
 (segment (start 171.45 90.4875) (end 171.45 85.725) (width 0.25) (layer "F.Cu") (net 8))
 (segment (start 165.1 94.615) (end 165.1 90.4875) (width 0.25) (layer "F.Cu") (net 8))
 (via (at 171.45 90.4875) (size 0.8) (drill 0.4) (layers "F.Cu" "B.Cu") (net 8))
 (via (at 165.1 90.4875) (size 0.8) (drill 0.4) (layers "F.Cu" "B.Cu") (free) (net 8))
 (via (at 171.45 85.725) (size 0.8) (drill 0.4) (layers "F.Cu" "B.Cu") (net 8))
 (segment (start 171.45 90.4875) (end 165.1 90.4875) (width 0.25) (layer "B.Cu") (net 8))
 (segment (start 171.45 85.725) (end 178.025 85.725) (width 0.25) (layer "B.Cu") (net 8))
 (segment (start 178.025 85.725) (end 180.975 82.775) (width 0.25) (layer "B.Cu") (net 8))
 (segment (start 76.2 123.825) (end 76.2 85.725) (width 0.25) (layer "B.Cu") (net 10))
 (segment (start 127 94.615) (end 127 90.4875) (width 0.25) (layer "F.Cu") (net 9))
 (segment (start 120.65 90.4875) (end 120.65 85.725) (width 0.25) (layer "F.Cu") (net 9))
 (segment (start 120.65 94.615) (end 120.65 90.4875) (width 0.25) (layer "F.Cu") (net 9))
 (via (at 127 90.4875) (size 0.8) (drill 0.4) (layers "F.Cu" "B.Cu") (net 9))
 (via (at 120.65 90.4875) (size 0.8) (drill 0.4) (layers "F.Cu" "B.Cu") (free) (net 9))
 (segment (start 120.65 90.4875) (end 127 90.4875) (width 0.25) (layer "B.Cu") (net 9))
 (segment (start 120.65 114.935) (end 120.65 119.0625) (width 0.25) (layer "F.Cu") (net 13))
 (segment (start 120.65 119.0625) (end 120.65 123.825) (width 0.25) (layer "F.Cu") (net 13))
 (via (at 120.65 119.0625) (size 0.8) (drill 0.4) (layers "F.Cu" "B.Cu") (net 13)))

